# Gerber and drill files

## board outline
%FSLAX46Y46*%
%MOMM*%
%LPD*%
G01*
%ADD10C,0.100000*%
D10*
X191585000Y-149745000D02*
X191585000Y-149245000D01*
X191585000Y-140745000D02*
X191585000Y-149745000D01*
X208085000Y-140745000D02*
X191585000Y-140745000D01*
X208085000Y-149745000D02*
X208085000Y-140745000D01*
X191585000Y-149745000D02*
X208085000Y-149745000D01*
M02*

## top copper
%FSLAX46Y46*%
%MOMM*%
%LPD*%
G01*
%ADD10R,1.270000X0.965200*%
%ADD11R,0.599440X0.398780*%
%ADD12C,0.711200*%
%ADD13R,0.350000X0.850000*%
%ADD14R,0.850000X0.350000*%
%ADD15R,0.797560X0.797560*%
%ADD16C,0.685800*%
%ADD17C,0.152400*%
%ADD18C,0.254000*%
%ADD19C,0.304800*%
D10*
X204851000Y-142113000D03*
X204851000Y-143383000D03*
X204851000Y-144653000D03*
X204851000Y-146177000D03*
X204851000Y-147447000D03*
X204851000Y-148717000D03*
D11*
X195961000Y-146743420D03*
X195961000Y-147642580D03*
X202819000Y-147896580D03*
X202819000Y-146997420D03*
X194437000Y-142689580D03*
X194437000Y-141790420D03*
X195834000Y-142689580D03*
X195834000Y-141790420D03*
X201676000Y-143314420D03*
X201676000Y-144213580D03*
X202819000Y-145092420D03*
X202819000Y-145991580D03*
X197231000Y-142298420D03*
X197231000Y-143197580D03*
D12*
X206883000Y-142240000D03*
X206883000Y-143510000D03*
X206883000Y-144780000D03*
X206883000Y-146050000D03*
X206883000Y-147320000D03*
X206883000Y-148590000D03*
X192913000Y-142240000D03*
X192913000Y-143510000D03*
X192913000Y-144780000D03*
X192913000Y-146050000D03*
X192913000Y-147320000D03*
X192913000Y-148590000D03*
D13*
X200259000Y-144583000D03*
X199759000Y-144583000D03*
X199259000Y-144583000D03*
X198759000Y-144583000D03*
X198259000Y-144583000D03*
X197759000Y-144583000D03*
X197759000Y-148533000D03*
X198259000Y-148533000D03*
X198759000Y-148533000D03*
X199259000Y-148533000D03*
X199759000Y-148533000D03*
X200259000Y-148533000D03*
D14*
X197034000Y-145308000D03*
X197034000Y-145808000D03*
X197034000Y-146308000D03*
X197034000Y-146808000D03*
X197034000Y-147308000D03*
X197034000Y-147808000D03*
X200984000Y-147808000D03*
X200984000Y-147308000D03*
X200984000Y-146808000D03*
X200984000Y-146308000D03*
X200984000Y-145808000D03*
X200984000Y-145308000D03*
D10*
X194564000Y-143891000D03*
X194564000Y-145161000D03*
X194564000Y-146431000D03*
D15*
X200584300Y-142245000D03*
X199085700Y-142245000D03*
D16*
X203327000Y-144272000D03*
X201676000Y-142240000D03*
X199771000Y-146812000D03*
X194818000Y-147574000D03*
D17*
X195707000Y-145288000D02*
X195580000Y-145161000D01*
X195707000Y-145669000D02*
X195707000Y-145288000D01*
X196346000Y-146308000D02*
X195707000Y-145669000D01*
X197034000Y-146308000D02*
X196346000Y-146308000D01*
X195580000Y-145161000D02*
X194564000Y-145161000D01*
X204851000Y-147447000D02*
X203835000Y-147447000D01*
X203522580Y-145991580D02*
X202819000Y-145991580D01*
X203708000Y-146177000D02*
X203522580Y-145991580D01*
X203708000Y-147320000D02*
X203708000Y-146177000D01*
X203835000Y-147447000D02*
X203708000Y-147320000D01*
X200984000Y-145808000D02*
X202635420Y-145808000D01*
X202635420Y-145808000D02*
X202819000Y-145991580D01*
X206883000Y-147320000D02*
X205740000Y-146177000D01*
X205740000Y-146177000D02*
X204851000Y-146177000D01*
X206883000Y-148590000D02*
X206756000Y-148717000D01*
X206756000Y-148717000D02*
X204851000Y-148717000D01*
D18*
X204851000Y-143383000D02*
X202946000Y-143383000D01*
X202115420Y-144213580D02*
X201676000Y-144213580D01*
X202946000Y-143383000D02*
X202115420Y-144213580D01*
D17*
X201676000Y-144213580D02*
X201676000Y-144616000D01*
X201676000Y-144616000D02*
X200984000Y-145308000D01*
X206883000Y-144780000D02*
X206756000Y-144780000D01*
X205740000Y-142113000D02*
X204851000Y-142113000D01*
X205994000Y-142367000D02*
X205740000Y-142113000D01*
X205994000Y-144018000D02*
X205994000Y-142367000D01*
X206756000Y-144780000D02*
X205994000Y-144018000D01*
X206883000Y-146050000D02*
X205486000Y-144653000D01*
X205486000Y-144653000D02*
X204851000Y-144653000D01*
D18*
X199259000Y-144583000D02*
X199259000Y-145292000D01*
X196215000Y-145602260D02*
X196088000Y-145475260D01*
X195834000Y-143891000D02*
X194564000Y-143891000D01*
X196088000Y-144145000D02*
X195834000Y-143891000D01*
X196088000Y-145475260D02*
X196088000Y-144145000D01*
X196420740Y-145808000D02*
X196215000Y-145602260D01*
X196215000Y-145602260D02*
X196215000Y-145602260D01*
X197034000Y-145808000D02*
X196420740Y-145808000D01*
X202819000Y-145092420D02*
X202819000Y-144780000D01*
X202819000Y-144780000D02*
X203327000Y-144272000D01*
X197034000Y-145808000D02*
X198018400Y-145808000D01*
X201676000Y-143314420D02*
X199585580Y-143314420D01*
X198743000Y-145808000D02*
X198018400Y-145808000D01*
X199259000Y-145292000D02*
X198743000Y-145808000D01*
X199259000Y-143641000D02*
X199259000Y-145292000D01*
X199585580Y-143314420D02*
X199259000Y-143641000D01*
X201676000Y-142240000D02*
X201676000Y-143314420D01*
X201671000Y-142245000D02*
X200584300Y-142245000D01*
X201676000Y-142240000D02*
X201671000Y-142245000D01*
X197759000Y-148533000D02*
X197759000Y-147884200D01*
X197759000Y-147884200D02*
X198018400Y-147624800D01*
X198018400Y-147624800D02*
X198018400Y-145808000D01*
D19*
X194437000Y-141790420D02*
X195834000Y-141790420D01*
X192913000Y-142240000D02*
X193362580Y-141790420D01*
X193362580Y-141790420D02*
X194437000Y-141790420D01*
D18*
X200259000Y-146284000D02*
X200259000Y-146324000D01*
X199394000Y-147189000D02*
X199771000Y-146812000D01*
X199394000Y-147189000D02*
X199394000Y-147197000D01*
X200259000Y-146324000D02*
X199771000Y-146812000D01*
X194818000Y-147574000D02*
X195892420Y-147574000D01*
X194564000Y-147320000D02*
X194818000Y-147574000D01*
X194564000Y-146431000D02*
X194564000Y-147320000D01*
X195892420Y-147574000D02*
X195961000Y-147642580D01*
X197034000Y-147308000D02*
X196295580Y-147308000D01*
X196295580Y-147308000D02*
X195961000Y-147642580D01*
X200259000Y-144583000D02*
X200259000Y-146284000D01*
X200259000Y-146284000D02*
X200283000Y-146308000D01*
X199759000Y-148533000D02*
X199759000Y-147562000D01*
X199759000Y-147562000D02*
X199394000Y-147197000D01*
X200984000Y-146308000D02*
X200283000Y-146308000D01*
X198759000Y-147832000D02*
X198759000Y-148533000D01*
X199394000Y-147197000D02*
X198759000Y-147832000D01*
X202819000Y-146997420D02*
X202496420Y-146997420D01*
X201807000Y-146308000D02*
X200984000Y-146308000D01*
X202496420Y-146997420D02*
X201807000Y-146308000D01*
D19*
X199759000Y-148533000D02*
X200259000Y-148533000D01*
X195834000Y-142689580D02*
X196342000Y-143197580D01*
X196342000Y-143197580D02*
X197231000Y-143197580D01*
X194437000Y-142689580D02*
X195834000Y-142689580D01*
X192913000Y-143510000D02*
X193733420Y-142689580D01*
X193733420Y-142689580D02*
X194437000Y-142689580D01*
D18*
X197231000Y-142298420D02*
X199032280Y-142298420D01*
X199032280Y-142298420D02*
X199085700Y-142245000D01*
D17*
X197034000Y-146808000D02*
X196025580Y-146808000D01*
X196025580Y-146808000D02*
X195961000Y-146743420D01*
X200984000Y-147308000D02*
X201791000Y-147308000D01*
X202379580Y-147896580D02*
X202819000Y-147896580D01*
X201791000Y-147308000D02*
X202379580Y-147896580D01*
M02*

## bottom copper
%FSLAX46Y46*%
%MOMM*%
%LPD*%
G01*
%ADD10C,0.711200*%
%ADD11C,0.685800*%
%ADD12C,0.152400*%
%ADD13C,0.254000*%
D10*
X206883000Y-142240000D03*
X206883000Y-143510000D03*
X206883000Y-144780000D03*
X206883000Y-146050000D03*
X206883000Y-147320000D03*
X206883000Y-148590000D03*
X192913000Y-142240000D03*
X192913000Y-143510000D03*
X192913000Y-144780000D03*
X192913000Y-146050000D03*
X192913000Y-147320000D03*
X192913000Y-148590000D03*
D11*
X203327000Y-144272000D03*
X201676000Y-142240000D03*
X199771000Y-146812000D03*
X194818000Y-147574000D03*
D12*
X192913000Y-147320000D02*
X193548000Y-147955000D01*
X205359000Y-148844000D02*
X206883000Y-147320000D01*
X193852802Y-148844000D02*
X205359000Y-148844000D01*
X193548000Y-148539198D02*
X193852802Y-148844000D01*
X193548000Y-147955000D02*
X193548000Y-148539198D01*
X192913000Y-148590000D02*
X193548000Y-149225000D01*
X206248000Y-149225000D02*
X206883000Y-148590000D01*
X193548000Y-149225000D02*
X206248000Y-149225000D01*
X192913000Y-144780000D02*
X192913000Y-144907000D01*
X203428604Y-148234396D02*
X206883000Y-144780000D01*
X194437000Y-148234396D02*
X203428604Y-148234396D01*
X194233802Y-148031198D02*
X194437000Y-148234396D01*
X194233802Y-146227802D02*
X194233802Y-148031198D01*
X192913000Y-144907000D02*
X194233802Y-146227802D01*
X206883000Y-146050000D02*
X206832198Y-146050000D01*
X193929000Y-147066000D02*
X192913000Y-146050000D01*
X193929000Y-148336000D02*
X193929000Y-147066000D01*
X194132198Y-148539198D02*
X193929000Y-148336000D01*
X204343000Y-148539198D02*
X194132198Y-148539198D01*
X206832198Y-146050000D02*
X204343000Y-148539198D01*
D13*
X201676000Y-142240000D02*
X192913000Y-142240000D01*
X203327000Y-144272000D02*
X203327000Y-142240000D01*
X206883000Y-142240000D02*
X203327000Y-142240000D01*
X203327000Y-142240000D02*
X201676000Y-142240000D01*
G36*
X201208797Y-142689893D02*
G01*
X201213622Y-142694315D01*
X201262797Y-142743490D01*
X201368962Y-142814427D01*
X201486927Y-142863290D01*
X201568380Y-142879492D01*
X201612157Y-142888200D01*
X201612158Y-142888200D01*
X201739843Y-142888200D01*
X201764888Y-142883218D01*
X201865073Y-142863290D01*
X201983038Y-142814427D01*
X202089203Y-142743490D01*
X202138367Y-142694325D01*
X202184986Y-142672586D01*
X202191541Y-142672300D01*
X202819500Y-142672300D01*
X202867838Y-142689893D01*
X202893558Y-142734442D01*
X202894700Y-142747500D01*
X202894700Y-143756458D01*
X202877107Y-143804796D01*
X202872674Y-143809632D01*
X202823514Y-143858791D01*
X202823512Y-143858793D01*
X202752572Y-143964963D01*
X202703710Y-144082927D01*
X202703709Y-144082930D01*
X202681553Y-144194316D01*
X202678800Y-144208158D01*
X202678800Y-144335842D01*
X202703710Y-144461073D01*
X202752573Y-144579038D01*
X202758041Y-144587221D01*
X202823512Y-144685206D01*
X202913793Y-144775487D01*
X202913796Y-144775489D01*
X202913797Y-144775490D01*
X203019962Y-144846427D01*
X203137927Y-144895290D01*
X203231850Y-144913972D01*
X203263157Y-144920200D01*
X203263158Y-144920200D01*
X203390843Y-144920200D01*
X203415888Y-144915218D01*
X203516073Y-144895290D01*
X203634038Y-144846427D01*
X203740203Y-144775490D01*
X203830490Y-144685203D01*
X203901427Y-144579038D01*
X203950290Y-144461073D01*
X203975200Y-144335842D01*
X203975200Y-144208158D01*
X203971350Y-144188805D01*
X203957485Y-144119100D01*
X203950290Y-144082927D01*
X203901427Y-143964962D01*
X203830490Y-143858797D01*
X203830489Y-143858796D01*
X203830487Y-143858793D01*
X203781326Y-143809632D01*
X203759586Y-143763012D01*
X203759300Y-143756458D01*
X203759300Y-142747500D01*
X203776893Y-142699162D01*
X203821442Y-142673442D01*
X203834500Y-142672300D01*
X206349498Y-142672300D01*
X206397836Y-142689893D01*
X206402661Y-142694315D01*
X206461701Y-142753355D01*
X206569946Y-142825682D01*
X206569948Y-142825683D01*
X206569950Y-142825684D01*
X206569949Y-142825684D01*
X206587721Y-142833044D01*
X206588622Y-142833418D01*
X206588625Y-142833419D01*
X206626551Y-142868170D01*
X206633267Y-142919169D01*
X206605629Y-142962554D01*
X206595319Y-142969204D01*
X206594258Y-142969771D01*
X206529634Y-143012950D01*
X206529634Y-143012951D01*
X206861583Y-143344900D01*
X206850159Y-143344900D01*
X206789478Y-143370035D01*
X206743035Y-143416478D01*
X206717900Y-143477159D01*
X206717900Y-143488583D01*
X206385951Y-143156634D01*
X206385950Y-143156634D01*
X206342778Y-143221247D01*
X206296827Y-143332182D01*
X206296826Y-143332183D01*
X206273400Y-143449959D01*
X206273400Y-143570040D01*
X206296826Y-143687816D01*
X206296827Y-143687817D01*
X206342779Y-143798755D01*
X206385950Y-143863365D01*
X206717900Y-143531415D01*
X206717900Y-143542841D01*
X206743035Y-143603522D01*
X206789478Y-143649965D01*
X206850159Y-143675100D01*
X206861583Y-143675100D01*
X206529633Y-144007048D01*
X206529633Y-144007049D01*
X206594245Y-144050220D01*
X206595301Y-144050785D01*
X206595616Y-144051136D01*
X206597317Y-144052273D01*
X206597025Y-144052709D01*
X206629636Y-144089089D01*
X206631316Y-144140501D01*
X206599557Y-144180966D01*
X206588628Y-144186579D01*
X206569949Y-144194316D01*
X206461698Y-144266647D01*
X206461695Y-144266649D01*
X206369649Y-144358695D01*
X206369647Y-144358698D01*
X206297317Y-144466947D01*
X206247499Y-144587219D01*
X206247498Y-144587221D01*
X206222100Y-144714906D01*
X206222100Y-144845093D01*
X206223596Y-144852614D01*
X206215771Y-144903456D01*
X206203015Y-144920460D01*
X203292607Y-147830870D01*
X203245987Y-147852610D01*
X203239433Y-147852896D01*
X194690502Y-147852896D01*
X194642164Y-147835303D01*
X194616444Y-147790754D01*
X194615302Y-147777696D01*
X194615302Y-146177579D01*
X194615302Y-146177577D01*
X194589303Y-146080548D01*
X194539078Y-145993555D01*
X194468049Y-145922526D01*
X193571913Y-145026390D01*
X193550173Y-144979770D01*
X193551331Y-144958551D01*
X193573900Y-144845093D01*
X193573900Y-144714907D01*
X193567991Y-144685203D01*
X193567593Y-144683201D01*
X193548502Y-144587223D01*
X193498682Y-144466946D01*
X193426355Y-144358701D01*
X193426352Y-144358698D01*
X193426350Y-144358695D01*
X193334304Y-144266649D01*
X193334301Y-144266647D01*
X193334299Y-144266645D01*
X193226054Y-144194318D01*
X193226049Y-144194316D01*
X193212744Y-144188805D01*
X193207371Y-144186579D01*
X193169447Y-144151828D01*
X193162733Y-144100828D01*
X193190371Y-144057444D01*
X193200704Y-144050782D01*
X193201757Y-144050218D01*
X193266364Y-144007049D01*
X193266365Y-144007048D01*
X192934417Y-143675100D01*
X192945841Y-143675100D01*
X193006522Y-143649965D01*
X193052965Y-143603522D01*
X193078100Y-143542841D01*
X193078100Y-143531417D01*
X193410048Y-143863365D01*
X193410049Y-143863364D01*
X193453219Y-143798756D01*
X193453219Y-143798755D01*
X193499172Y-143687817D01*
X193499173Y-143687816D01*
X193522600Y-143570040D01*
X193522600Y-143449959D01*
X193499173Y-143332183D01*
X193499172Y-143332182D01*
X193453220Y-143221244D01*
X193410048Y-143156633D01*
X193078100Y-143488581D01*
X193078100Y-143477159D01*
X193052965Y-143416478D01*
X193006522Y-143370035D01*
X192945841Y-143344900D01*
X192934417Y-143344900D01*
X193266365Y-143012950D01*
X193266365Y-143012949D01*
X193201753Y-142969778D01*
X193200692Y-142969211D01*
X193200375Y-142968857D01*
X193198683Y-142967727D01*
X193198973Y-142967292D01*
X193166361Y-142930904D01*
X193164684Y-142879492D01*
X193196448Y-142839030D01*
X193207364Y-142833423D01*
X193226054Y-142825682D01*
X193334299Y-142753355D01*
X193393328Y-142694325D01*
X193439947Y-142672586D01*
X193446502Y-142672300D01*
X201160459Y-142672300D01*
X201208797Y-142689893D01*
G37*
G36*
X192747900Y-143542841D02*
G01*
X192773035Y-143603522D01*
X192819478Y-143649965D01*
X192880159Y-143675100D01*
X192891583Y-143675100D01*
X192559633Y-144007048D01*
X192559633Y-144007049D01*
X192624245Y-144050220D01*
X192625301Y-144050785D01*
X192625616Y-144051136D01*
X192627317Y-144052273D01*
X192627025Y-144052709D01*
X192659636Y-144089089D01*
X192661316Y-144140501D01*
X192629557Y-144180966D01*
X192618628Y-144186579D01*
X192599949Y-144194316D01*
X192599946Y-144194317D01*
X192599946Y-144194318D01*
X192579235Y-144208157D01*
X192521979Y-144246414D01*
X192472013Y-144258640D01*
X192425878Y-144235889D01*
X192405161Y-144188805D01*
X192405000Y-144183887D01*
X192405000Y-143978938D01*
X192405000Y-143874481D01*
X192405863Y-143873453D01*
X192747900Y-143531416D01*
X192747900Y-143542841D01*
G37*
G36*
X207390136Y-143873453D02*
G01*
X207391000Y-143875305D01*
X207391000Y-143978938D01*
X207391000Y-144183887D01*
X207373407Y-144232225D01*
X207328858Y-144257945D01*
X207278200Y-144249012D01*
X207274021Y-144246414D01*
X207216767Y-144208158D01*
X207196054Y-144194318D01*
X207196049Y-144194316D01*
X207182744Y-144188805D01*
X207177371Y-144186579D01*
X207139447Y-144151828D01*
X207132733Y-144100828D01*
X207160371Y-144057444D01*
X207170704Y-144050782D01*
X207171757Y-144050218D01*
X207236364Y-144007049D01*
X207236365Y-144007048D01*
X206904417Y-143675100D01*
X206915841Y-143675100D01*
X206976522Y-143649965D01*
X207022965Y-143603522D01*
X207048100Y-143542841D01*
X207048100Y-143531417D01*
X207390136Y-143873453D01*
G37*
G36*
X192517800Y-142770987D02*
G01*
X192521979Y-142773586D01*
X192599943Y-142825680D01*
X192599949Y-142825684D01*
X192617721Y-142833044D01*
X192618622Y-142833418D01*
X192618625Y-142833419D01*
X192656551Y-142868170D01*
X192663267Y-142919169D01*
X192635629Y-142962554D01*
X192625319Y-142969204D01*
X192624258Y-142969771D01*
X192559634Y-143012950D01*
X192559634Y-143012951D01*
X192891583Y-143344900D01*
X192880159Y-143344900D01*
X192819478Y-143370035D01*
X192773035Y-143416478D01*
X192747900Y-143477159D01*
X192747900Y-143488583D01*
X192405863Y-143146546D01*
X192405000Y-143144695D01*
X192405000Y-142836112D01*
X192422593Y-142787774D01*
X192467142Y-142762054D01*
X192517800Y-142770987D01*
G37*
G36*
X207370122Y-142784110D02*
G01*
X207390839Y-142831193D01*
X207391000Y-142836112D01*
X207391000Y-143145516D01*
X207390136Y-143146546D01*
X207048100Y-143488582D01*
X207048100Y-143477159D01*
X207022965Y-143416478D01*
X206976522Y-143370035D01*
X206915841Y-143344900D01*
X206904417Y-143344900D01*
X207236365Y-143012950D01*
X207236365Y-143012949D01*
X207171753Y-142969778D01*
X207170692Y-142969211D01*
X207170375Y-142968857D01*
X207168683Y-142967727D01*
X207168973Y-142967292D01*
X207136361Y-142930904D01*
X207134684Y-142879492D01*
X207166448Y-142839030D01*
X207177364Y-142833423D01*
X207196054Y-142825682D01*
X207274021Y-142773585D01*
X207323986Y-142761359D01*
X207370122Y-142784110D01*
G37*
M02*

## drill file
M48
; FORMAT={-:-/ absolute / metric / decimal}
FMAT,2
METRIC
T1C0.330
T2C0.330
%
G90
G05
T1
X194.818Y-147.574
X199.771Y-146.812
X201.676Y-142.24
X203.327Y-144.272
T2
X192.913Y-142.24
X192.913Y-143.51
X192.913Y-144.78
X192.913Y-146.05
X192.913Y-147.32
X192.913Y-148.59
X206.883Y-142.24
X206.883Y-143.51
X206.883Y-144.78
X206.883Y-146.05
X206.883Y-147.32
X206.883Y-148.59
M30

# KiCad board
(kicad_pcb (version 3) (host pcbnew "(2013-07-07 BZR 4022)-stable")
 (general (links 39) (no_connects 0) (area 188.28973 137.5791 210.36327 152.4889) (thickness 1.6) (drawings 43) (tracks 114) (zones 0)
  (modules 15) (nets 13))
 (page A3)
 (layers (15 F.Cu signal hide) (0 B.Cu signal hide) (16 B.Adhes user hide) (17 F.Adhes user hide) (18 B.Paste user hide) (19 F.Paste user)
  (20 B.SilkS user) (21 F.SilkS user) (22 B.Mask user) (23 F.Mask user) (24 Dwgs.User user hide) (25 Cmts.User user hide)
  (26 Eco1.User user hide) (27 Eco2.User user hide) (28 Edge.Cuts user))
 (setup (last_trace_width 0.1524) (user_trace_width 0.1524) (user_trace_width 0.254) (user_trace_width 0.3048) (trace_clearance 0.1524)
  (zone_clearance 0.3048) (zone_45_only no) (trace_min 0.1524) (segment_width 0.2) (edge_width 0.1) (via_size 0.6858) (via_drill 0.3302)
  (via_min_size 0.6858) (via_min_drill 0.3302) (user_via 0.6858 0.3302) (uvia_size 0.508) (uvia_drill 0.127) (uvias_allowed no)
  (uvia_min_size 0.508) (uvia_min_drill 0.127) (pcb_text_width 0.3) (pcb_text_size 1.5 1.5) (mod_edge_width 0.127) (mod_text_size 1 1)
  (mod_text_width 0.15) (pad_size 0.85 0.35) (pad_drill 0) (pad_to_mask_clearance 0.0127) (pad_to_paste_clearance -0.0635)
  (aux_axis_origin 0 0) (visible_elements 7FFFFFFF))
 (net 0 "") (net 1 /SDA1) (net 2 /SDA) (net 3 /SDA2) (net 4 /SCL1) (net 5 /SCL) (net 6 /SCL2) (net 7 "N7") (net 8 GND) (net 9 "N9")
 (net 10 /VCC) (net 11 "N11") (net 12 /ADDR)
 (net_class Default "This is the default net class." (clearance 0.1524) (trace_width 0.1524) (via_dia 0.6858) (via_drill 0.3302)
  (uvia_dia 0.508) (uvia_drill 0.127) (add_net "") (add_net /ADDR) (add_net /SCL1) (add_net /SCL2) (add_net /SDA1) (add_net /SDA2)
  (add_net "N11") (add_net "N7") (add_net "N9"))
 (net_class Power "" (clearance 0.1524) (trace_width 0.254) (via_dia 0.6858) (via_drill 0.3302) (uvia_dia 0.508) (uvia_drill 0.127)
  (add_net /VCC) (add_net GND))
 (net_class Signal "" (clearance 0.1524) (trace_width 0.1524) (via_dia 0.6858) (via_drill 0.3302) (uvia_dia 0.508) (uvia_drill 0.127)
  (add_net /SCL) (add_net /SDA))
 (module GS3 (layer F.Cu) (at 204.851 143.383)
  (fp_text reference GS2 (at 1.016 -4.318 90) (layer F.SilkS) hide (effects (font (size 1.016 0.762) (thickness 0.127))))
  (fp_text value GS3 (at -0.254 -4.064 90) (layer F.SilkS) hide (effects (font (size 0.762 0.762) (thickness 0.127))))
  (pad 1 smd rect (at 0 -1.27) (size 1.27 0.9652) (layers F.Cu F.Paste F.Mask) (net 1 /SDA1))
  (pad 2 smd rect (at 0 0) (size 1.27 0.9652) (layers F.Cu F.Paste F.Mask) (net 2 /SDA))
  (pad 3 smd rect (at 0 1.27) (size 1.27 0.9652) (layers F.Cu F.Paste F.Mask) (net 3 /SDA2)))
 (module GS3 (layer F.Cu) (at 204.851 147.447)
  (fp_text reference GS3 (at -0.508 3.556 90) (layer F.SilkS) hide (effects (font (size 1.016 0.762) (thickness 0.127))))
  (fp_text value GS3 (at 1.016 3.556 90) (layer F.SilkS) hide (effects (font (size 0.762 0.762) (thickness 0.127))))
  (pad 1 smd rect (at 0 -1.27) (size 1.27 0.9652) (layers F.Cu F.Paste F.Mask) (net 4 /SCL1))
  (pad 2 smd rect (at 0 0) (size 1.27 0.9652) (layers F.Cu F.Paste F.Mask) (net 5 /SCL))
  (pad 3 smd rect (at 0 1.27) (size 1.27 0.9652) (layers F.Cu F.Paste F.Mask) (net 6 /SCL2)))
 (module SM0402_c (layer F.Cu) (at 195.961 147.193 270)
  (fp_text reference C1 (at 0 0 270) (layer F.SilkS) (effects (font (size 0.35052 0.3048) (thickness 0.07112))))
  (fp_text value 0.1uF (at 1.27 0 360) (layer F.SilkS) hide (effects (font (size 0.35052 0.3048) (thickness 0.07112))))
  (pad 1 smd rect (at -0.44958 0 270) (size 0.39878 0.59944) (layers F.Cu F.Paste F.Mask) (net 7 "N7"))
  (pad 2 smd rect (at 0.44958 0 270) (size 0.39878 0.59944) (layers F.Cu F.Paste F.Mask) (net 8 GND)))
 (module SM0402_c (layer F.Cu) (at 202.819 147.447 90)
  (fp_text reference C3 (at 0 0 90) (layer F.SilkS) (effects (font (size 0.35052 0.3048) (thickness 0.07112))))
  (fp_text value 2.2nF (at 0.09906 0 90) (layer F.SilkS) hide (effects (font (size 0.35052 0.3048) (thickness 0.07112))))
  (pad 1 smd rect (at -0.44958 0 90) (size 0.39878 0.59944) (layers F.Cu F.Paste F.Mask) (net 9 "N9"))
  (pad 2 smd rect (at 0.44958 0 90) (size 0.39878 0.59944) (layers F.Cu F.Paste F.Mask) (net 8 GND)))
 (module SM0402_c (layer F.Cu) (at 194.437 142.24 90)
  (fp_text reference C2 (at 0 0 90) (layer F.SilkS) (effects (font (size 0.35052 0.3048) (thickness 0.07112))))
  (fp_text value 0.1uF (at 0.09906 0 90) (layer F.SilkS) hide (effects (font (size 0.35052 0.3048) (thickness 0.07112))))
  (pad 1 smd rect (at -0.44958 0 90) (size 0.39878 0.59944) (layers F.Cu F.Paste F.Mask) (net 8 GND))
  (pad 2 smd rect (at 0.44958 0 90) (size 0.39878 0.59944) (layers F.Cu F.Paste F.Mask) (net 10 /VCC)))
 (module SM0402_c (layer F.Cu) (at 195.834 142.24 90)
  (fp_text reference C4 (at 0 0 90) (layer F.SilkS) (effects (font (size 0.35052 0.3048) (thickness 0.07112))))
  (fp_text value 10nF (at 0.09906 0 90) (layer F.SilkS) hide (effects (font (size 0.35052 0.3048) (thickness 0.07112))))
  (pad 1 smd rect (at -0.44958 0 90) (size 0.39878 0.59944) (layers F.Cu F.Paste F.Mask) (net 8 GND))
  (pad 2 smd rect (at 0.44958 0 90) (size 0.39878 0.59944) (layers F.Cu F.Paste F.Mask) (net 10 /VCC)))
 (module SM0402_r (layer F.Cu) (at 201.676 143.764 270)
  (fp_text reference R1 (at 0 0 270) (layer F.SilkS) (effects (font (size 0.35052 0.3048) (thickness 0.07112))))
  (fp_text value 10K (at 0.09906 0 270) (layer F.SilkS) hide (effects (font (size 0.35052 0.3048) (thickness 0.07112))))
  (pad 1 smd rect (at -0.44958 0 270) (size 0.39878 0.59944) (layers F.Cu F.Paste F.Mask) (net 10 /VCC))
  (pad 2 smd rect (at 0.44958 0 270) (size 0.39878 0.59944) (layers F.Cu F.Paste F.Mask) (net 2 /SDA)))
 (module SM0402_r (layer F.Cu) (at 202.819 145.542 270)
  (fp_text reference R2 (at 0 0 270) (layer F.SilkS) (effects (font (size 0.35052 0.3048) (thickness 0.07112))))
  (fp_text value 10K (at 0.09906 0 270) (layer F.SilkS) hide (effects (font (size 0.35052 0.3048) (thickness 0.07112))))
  (pad 1 smd rect (at -0.44958 0 270) (size 0.39878 0.59944) (layers F.Cu F.Paste F.Mask) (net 10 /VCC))
  (pad 2 smd rect (at 0.44958 0 270) (size 0.39878 0.59944) (layers F.Cu F.Paste F.Mask) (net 5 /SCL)))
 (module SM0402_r (layer F.Cu) (at 197.231 142.748 270)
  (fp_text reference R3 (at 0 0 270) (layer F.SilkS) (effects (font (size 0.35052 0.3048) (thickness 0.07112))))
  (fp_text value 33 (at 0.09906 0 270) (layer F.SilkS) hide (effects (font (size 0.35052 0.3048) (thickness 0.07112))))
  (pad 1 smd rect (at -0.44958 0 270) (size 0.39878 0.59944) (layers F.Cu F.Paste F.Mask) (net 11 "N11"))
  (pad 2 smd rect (at 0.44958 0 270) (size 0.39878 0.59944) (layers F.Cu F.Paste F.Mask) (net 8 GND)))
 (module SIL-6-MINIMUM (layer F.Cu) (at 206.883 145.415 270)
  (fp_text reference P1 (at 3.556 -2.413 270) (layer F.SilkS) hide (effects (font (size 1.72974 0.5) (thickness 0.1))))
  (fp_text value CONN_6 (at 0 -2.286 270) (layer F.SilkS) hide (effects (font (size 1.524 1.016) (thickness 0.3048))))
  (pad 1 thru_hole circle (at -3.175 0 270) (size 0.7112 0.7112) (drill 0.3302) (layers *.Cu *.Mask F.SilkS) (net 10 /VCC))
  (pad 2 thru_hole circle (at -1.905 0 270) (size 0.7112 0.7112) (drill 0.3302) (layers *.Cu *.Mask F.SilkS) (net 8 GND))
  (pad 3 thru_hole circle (at -0.635 0 270) (size 0.7112 0.7112) (drill 0.3302) (layers *.Cu *.Mask F.SilkS) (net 1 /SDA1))
  (pad 4 thru_hole circle (at 0.635 0 270) (size 0.7112 0.7112) (drill 0.3302) (layers *.Cu *.Mask F.SilkS) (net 3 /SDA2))
  (pad 5 thru_hole circle (at 1.905 0 270) (size 0.7112 0.7112) (drill 0.3302) (layers *.Cu *.Mask F.SilkS) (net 4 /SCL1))
  (pad 6 thru_hole circle (at 3.175 0 270) (size 0.7112 0.7112) (drill 0.3302) (layers *.Cu *.Mask F.SilkS) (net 6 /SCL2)))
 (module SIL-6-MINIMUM (layer F.Cu) (at 192.913 145.415 270)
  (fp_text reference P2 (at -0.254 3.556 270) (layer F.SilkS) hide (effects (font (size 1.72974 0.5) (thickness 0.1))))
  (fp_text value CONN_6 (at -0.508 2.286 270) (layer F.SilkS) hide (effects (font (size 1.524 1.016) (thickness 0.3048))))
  (pad 1 thru_hole circle (at -3.175 0 270) (size 0.7112 0.7112) (drill 0.3302) (layers *.Cu *.Mask F.SilkS) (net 10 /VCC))
  (pad 2 thru_hole circle (at -1.905 0 270) (size 0.7112 0.7112) (drill 0.3302) (layers *.Cu *.Mask F.SilkS) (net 8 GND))
  (pad 3 thru_hole circle (at -0.635 0 270) (size 0.7112 0.7112) (drill 0.3302) (layers *.Cu *.Mask F.SilkS) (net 1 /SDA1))
  (pad 4 thru_hole circle (at 0.635 0 270) (size 0.7112 0.7112) (drill 0.3302) (layers *.Cu *.Mask F.SilkS) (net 3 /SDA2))
  (pad 5 thru_hole circle (at 1.905 0 270) (size 0.7112 0.7112) (drill 0.3302) (layers *.Cu *.Mask F.SilkS) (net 4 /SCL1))
  (pad 6 thru_hole circle (at 3.175 0 270) (size 0.7112 0.7112) (drill 0.3302) (layers *.Cu *.Mask F.SilkS) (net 6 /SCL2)))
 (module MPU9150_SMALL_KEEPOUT (layer F.Cu) (at 199.009 146.558 270)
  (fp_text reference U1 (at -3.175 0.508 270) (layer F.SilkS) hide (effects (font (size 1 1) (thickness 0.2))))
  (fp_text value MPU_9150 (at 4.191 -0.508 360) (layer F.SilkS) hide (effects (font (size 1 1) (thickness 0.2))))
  (pad 1 smd rect (at -1.975 -1.25 270) (size 0.85 0.35) (layers F.Cu F.Paste F.Mask) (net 8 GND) (clearance 0.0762))
  (pad 2 smd rect (at -1.975 -0.75 270) (size 0.85 0.35) (layers F.Cu F.Paste F.Mask) (clearance 0.0762))
  (pad 3 smd rect (at -1.975 -0.25 270) (size 0.85 0.35) (layers F.Cu F.Paste F.Mask) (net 10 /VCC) (clearance 0.0762))
  (pad 4 smd rect (at -1.975 0.25 270) (size 0.85 0.35) (layers F.Cu F.Paste F.Mask) (clearance 0.0762))
  (pad 5 smd rect (at -1.975 0.75 270) (size 0.85 0.35) (layers F.Cu F.Paste F.Mask) (clearance 0.0762))
  (pad 6 smd rect (at -1.975 1.25 270) (size 0.85 0.35) (layers F.Cu F.Paste F.Mask) (clearance 0.0762))
  (pad 13 smd rect (at 1.975 1.25 270) (size 0.85 0.35) (layers F.Cu F.Paste F.Mask) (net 10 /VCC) (clearance 0.0762))
  (pad 14 smd rect (at 1.975 0.75 270) (size 0.85 0.35) (layers F.Cu F.Paste F.Mask) (clearance 0.0762))
  (pad 15 smd rect (at 1.975 0.25 270) (size 0.85 0.35) (layers F.Cu F.Paste F.Mask) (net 8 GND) (clearance 0.0762))
  (pad 16 smd rect (at 1.975 -0.25 270) (size 0.85 0.35) (layers F.Cu F.Paste F.Mask) (clearance 0.0762))
  (pad 17 smd rect (at 1.975 -0.75 270) (size 0.85 0.35) (layers F.Cu F.Paste F.Mask) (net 8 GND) (clearance 0.0762))
  (pad 18 smd rect (at 1.975 -1.25 270) (size 0.85 0.35) (layers F.Cu F.Paste F.Mask) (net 8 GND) (clearance 0.0762))
  (pad 7 smd rect (at -1.25 1.975 270) (size 0.35 0.85) (layers F.Cu F.Paste F.Mask) (clearance 0.0762))
  (pad 8 smd rect (at -0.75 1.975 270) (size 0.35 0.85) (layers F.Cu F.Paste F.Mask) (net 10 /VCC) (clearance 0.0762))
  (pad 9 smd rect (at -0.25 1.975 270) (size 0.35 0.85) (layers F.Cu F.Paste F.Mask) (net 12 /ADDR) (clearance 0.0762))
  (pad 10 smd rect (at 0.25 1.975 270) (size 0.35 0.85) (layers F.Cu F.Paste F.Mask) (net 7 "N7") (clearance 0.0762))
  (pad 11 smd rect (at 0.75 1.975 270) (size 0.35 0.85) (layers F.Cu F.Paste F.Mask) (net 8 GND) (clearance 0.0762))
  (pad 12 smd rect (at 1.25 1.975 270) (size 0.35 0.85) (layers F.Cu F.Paste F.Mask) (clearance 0.0762))
  (pad 19 smd rect (at 1.25 -1.975 270) (size 0.35 0.85) (layers F.Cu F.Paste F.Mask) (clearance 0.0762))
  (pad 20 smd rect (at 0.75 -1.975 270) (size 0.35 0.85) (layers F.Cu F.Paste F.Mask) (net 9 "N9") (clearance 0.0762))
  (pad 21 smd rect (at 0.25 -1.975 270) (size 0.35 0.85) (layers F.Cu F.Paste F.Mask) (clearance 0.0762))
  (pad 22 smd rect (at -0.25 -1.975 270) (size 0.35 0.85) (layers F.Cu F.Paste F.Mask) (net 8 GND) (clearance 0.0762))
  (pad 23 smd rect (at -0.75 -1.975 270) (size 0.35 0.85) (layers F.Cu F.Paste F.Mask) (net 5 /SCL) (clearance 0.0762))
  (pad 24 smd rect (at -1.25 -1.975 270) (size 0.35 0.85) (layers F.Cu F.Paste F.Mask) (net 2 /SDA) (clearance 0.0762)))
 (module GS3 (layer F.Cu) (at 194.564 145.161)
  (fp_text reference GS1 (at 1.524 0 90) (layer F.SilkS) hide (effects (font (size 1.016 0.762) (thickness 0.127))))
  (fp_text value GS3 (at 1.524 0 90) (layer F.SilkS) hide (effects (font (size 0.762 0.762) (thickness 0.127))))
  (pad 1 smd rect (at 0 -1.27) (size 1.27 0.9652) (layers F.Cu F.Paste F.Mask) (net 10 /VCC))
  (pad 2 smd rect (at 0 0) (size 1.27 0.9652) (layers F.Cu F.Paste F.Mask) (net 12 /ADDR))
  (pad 3 smd rect (at 0 1.27) (size 1.27 0.9652) (layers F.Cu F.Paste F.Mask) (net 8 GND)))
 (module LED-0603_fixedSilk (layer F.Cu) (at 199.835 142.245 180)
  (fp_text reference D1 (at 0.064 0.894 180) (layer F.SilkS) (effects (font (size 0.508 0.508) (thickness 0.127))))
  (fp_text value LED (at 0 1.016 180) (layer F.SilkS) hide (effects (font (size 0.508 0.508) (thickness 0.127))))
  (pad 1 smd rect (at -0.7493 0 180) (size 0.79756 0.79756) (layers F.Cu F.Paste F.Mask) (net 10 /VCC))
  (pad 2 smd rect (at 0.7493 0 180) (size 0.79756 0.79756) (layers F.Cu F.Paste F.Mask) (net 11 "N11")))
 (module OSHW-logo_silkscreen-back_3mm (layer B.Cu) (at 197.485 147.701)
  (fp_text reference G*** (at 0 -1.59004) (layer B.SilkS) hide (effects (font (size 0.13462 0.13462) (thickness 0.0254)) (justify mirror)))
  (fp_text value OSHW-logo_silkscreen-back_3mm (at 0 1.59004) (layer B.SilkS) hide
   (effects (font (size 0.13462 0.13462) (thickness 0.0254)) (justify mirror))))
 (gr_line (start 191.585 149.745) (end 191.585 149.245) (angle 90) (layer Edge.Cuts) (width 0.1))
 (gr_line (start 191.585 140.745) (end 191.585 149.745) (angle 90) (layer Edge.Cuts) (width 0.1))
 (gr_line (start 208.085 140.745) (end 191.585 140.745) (angle 90) (layer Edge.Cuts) (width 0.1))
 (gr_line (start 208.085 149.745) (end 208.085 140.745) (angle 90) (layer Edge.Cuts) (width 0.1))
 (gr_line (start 191.585 149.745) (end 208.085 149.745) (angle 90) (layer Edge.Cuts) (width 0.1))
 (segment (start 195.707 145.288) (end 195.58 145.161) (width 0.1524) (layer F.Cu) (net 12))
 (segment (start 195.707 145.669) (end 195.707 145.288) (width 0.1524) (layer F.Cu) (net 12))
 (segment (start 196.346 146.308) (end 195.707 145.669) (width 0.1524) (layer F.Cu) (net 12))
 (segment (start 197.034 146.308) (end 196.346 146.308) (width 0.1524) (layer F.Cu) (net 12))
 (segment (start 195.58 145.161) (end 194.564 145.161) (width 0.1524) (layer F.Cu) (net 12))
 (segment (start 204.851 147.447) (end 203.835 147.447) (width 0.1524) (layer F.Cu) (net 5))
 (segment (start 203.52258 145.99158) (end 202.819 145.99158) (width 0.1524) (layer F.Cu) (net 5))
 (segment (start 203.708 146.177) (end 203.52258 145.99158) (width 0.1524) (layer F.Cu) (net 5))
 (segment (start 203.708 147.32) (end 203.708 146.177) (width 0.1524) (layer F.Cu) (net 5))
 (segment (start 203.835 147.447) (end 203.708 147.32) (width 0.1524) (layer F.Cu) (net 5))
 (segment (start 200.984 145.808) (end 202.63542 145.808) (width 0.1524) (layer F.Cu) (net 5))
 (segment (start 202.63542 145.808) (end 202.819 145.99158) (width 0.1524) (layer F.Cu) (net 5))
 (segment (start 192.913 147.32) (end 193.548 147.955) (width 0.1524) (layer B.Cu) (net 4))
 (segment (start 205.359 148.844) (end 206.883 147.32) (width 0.1524) (layer B.Cu) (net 4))
 (segment (start 193.852802 148.844) (end 205.359 148.844) (width 0.1524) (layer B.Cu) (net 4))
 (segment (start 193.548 148.539198) (end 193.852802 148.844) (width 0.1524) (layer B.Cu) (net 4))
 (segment (start 193.548 147.955) (end 193.548 148.539198) (width 0.1524) (layer B.Cu) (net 4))
 (segment (start 206.883 147.32) (end 205.74 146.177) (width 0.1524) (layer F.Cu) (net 4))
 (segment (start 205.74 146.177) (end 204.851 146.177) (width 0.1524) (layer F.Cu) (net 4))
 (segment (start 192.913 148.59) (end 193.548 149.225) (width 0.1524) (layer B.Cu) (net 6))
 (segment (start 206.248 149.225) (end 206.883 148.59) (width 0.1524) (layer B.Cu) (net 6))
 (segment (start 193.548 149.225) (end 206.248 149.225) (width 0.1524) (layer B.Cu) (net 6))
 (segment (start 206.883 148.59) (end 206.756 148.717) (width 0.1524) (layer F.Cu) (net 6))
 (segment (start 206.756 148.717) (end 204.851 148.717) (width 0.1524) (layer F.Cu) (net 6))
 (segment (start 204.851 143.383) (end 202.946 143.383) (width 0.254) (layer F.Cu) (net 2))
 (segment (start 202.11542 144.21358) (end 201.676 144.21358) (width 0.254) (layer F.Cu) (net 2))
 (segment (start 202.946 143.383) (end 202.11542 144.21358) (width 0.254) (layer F.Cu) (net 2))
 (segment (start 201.676 144.21358) (end 201.676 144.616) (width 0.1524) (layer F.Cu) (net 2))
 (segment (start 201.676 144.616) (end 200.984 145.308) (width 0.1524) (layer F.Cu) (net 2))
 (segment (start 192.913 144.78) (end 192.913 144.907) (width 0.1524) (layer B.Cu) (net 1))
 (segment (start 203.428604 148.234396) (end 206.883 144.78) (width 0.1524) (layer B.Cu) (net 1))
 (segment (start 194.437 148.234396) (end 203.428604 148.234396) (width 0.1524) (layer B.Cu) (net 1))
 (segment (start 194.233802 148.031198) (end 194.437 148.234396) (width 0.1524) (layer B.Cu) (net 1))
 (segment (start 194.233802 146.227802) (end 194.233802 148.031198) (width 0.1524) (layer B.Cu) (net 1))
 (segment (start 192.913 144.907) (end 194.233802 146.227802) (width 0.1524) (layer B.Cu) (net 1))
 (segment (start 206.883 144.78) (end 206.756 144.78) (width 0.1524) (layer F.Cu) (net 1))
 (segment (start 205.74 142.113) (end 204.851 142.113) (width 0.1524) (layer F.Cu) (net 1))
 (segment (start 205.994 142.367) (end 205.74 142.113) (width 0.1524) (layer F.Cu) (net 1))
 (segment (start 205.994 144.018) (end 205.994 142.367) (width 0.1524) (layer F.Cu) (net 1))
 (segment (start 206.756 144.78) (end 205.994 144.018) (width 0.1524) (layer F.Cu) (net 1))
 (segment (start 206.883 146.05) (end 206.832198 146.05) (width 0.1524) (layer B.Cu) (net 3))
 (segment (start 193.929 147.066) (end 192.913 146.05) (width 0.1524) (layer B.Cu) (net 3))
 (segment (start 193.929 148.336) (end 193.929 147.066) (width 0.1524) (layer B.Cu) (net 3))
 (segment (start 194.132198 148.539198) (end 193.929 148.336) (width 0.1524) (layer B.Cu) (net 3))
 (segment (start 204.343 148.539198) (end 194.132198 148.539198) (width 0.1524) (layer B.Cu) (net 3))
 (segment (start 206.832198 146.05) (end 204.343 148.539198) (width 0.1524) (layer B.Cu) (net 3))
 (segment (start 206.883 146.05) (end 205.486 144.653) (width 0.1524) (layer F.Cu) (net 3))
 (segment (start 205.486 144.653) (end 204.851 144.653) (width 0.1524) (layer F.Cu) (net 3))
 (segment (start 199.259 144.583) (end 199.259 145.292) (width 0.254) (layer F.Cu) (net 10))
 (segment (start 196.215 145.60226) (end 196.088 145.47526) (width 0.254) (layer F.Cu) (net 10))
 (segment (start 195.834 143.891) (end 194.564 143.891) (width 0.254) (layer F.Cu) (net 10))
 (segment (start 196.088 144.145) (end 195.834 143.891) (width 0.254) (layer F.Cu) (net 10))
 (segment (start 196.088 145.47526) (end 196.088 144.145) (width 0.254) (layer F.Cu) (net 10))
 (segment (start 196.42074 145.808) (end 196.215 145.60226) (width 0.254) (layer F.Cu) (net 10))
 (segment (start 196.215 145.60226) (end 196.215 145.60226) (width 0.254) (layer F.Cu) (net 10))
 (segment (start 197.034 145.808) (end 196.42074 145.808) (width 0.254) (layer F.Cu) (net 10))
 (segment (start 201.676 142.24) (end 192.913 142.24) (width 0.254) (layer B.Cu) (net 10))
 (segment (start 202.819 145.09242) (end 202.819 144.78) (width 0.254) (layer F.Cu) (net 10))
 (segment (start 203.327 144.272) (end 203.327 142.24) (width 0.254) (layer B.Cu) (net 10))
 (via (at 203.327 144.272) (size 0.6858) (layers F.Cu B.Cu) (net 10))
 (segment (start 202.819 144.78) (end 203.327 144.272) (width 0.254) (layer F.Cu) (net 10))
 (segment (start 197.034 145.808) (end 198.0184 145.808) (width 0.254) (layer F.Cu) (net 10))
 (segment (start 201.676 143.31442) (end 199.58558 143.31442) (width 0.254) (layer F.Cu) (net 10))
 (segment (start 198.743 145.808) (end 198.0184 145.808) (width 0.254) (layer F.Cu) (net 10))
 (segment (start 199.259 145.292) (end 198.743 145.808) (width 0.254) (layer F.Cu) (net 10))
 (segment (start 199.259 143.641) (end 199.259 145.292) (width 0.254) (layer F.Cu) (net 10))
 (segment (start 199.58558 143.31442) (end 199.259 143.641) (width 0.254) (layer F.Cu) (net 10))
 (segment (start 201.676 142.24) (end 201.676 143.31442) (width 0.254) (layer F.Cu) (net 10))
 (segment (start 206.883 142.24) (end 203.327 142.24) (width 0.254) (layer B.Cu) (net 10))
 (segment (start 203.327 142.24) (end 201.676 142.24) (width 0.254) (layer B.Cu) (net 10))
 (segment (start 201.671 142.245) (end 200.5843 142.245) (width 0.254) (layer F.Cu) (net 10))
 (segment (start 201.676 142.24) (end 201.671 142.245) (width 0.254) (layer F.Cu) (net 10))
 (via (at 201.676 142.24) (size 0.6858) (layers F.Cu B.Cu) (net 10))
 (segment (start 197.759 148.533) (end 197.759 147.8842) (width 0.254) (layer F.Cu) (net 10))
 (segment (start 197.759 147.8842) (end 198.0184 147.6248) (width 0.254) (layer F.Cu) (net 10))
 (segment (start 198.0184 147.6248) (end 198.0184 145.808) (width 0.254) (layer F.Cu) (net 10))
 (segment (start 194.437 141.79042) (end 195.834 141.79042) (width 0.3048) (layer F.Cu) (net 10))
 (segment (start 192.913 142.24) (end 193.36258 141.79042) (width 0.3048) (layer F.Cu) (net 10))
 (segment (start 193.36258 141.79042) (end 194.437 141.79042) (width 0.3048) (layer F.Cu) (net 10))
 (segment (start 200.259 146.284) (end 200.259 146.324) (width 0.254) (layer F.Cu) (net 8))
 (segment (start 199.394 147.189) (end 199.771 146.812) (width 0.254) (layer F.Cu) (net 8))
 (via (at 199.771 146.812) (size 0.6858) (layers F.Cu B.Cu) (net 8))
 (segment (start 199.394 147.189) (end 199.394 147.197) (width 0.254) (layer F.Cu) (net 8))
 (segment (start 200.259 146.324) (end 199.771 146.812) (width 0.254) (layer F.Cu) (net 8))
 (segment (start 194.818 147.574) (end 195.89242 147.574) (width 0.254) (layer F.Cu) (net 8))
 (segment (start 194.564 147.32) (end 194.818 147.574) (width 0.254) (layer F.Cu) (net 8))
 (via (at 194.818 147.574) (size 0.6858) (layers F.Cu B.Cu) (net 8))
 (segment (start 194.564 146.431) (end 194.564 147.32) (width 0.254) (layer F.Cu) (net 8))
 (segment (start 195.89242 147.574) (end 195.961 147.64258) (width 0.254) (layer F.Cu) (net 8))
 (segment (start 197.034 147.308) (end 196.29558 147.308) (width 0.254) (layer F.Cu) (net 8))
 (segment (start 196.29558 147.308) (end 195.961 147.64258) (width 0.254) (layer F.Cu) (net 8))
 (segment (start 200.259 144.583) (end 200.259 146.284) (width 0.254) (layer F.Cu) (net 8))
 (segment (start 200.259 146.284) (end 200.283 146.308) (width 0.254) (layer F.Cu) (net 8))
 (segment (start 199.759 148.533) (end 199.759 147.562) (width 0.254) (layer F.Cu) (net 8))
 (segment (start 199.759 147.562) (end 199.394 147.197) (width 0.254) (layer F.Cu) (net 8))
 (segment (start 200.984 146.308) (end 200.283 146.308) (width 0.254) (layer F.Cu) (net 8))
 (segment (start 198.759 147.832) (end 198.759 148.533) (width 0.254) (layer F.Cu) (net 8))
 (segment (start 199.394 147.197) (end 198.759 147.832) (width 0.254) (layer F.Cu) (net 8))
 (segment (start 202.819 146.99742) (end 202.49642 146.99742) (width 0.254) (layer F.Cu) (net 8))
 (segment (start 201.807 146.308) (end 200.984 146.308) (width 0.254) (layer F.Cu) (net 8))
 (segment (start 202.49642 146.99742) (end 201.807 146.308) (width 0.254) (layer F.Cu) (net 8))
 (segment (start 199.759 148.533) (end 200.259 148.533) (width 0.3048) (layer F.Cu) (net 8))
 (segment (start 195.834 142.68958) (end 196.342 143.19758) (width 0.3048) (layer F.Cu) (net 8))
 (segment (start 196.342 143.19758) (end 197.231 143.19758) (width 0.3048) (layer F.Cu) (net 8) (status 20))
 (segment (start 194.437 142.68958) (end 195.834 142.68958) (width 0.3048) (layer F.Cu) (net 8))
 (segment (start 192.913 143.51) (end 193.73342 142.68958) (width 0.3048) (layer F.Cu) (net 8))
 (segment (start 193.73342 142.68958) (end 194.437 142.68958) (width 0.3048) (layer F.Cu) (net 8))
 (segment (start 197.231 142.29842) (end 199.03228 142.29842) (width 0.254) (layer F.Cu) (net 11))
 (segment (start 199.03228 142.29842) (end 199.0857 142.245) (width 0.254) (layer F.Cu) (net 11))
 (segment (start 197.034 146.808) (end 196.02558 146.808) (width 0.1524) (layer F.Cu) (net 7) (status 20))
 (segment (start 196.02558 146.808) (end 195.961 146.74342) (width 0.1524) (layer F.Cu) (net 7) (status 30))
 (segment (start 200.984 147.308) (end 201.791 147.308) (width 0.1524) (layer F.Cu) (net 9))
 (segment (start 202.37958 147.89658) (end 202.819 147.89658) (width 0.1524) (layer F.Cu) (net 9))
 (segment (start 201.791 147.308) (end 202.37958 147.89658) (width 0.1524) (layer F.Cu) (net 9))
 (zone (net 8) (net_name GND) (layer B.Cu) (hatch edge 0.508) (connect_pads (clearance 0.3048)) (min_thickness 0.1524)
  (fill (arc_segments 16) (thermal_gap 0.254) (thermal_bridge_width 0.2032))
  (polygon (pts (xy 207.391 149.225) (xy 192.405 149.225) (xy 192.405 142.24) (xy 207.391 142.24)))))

